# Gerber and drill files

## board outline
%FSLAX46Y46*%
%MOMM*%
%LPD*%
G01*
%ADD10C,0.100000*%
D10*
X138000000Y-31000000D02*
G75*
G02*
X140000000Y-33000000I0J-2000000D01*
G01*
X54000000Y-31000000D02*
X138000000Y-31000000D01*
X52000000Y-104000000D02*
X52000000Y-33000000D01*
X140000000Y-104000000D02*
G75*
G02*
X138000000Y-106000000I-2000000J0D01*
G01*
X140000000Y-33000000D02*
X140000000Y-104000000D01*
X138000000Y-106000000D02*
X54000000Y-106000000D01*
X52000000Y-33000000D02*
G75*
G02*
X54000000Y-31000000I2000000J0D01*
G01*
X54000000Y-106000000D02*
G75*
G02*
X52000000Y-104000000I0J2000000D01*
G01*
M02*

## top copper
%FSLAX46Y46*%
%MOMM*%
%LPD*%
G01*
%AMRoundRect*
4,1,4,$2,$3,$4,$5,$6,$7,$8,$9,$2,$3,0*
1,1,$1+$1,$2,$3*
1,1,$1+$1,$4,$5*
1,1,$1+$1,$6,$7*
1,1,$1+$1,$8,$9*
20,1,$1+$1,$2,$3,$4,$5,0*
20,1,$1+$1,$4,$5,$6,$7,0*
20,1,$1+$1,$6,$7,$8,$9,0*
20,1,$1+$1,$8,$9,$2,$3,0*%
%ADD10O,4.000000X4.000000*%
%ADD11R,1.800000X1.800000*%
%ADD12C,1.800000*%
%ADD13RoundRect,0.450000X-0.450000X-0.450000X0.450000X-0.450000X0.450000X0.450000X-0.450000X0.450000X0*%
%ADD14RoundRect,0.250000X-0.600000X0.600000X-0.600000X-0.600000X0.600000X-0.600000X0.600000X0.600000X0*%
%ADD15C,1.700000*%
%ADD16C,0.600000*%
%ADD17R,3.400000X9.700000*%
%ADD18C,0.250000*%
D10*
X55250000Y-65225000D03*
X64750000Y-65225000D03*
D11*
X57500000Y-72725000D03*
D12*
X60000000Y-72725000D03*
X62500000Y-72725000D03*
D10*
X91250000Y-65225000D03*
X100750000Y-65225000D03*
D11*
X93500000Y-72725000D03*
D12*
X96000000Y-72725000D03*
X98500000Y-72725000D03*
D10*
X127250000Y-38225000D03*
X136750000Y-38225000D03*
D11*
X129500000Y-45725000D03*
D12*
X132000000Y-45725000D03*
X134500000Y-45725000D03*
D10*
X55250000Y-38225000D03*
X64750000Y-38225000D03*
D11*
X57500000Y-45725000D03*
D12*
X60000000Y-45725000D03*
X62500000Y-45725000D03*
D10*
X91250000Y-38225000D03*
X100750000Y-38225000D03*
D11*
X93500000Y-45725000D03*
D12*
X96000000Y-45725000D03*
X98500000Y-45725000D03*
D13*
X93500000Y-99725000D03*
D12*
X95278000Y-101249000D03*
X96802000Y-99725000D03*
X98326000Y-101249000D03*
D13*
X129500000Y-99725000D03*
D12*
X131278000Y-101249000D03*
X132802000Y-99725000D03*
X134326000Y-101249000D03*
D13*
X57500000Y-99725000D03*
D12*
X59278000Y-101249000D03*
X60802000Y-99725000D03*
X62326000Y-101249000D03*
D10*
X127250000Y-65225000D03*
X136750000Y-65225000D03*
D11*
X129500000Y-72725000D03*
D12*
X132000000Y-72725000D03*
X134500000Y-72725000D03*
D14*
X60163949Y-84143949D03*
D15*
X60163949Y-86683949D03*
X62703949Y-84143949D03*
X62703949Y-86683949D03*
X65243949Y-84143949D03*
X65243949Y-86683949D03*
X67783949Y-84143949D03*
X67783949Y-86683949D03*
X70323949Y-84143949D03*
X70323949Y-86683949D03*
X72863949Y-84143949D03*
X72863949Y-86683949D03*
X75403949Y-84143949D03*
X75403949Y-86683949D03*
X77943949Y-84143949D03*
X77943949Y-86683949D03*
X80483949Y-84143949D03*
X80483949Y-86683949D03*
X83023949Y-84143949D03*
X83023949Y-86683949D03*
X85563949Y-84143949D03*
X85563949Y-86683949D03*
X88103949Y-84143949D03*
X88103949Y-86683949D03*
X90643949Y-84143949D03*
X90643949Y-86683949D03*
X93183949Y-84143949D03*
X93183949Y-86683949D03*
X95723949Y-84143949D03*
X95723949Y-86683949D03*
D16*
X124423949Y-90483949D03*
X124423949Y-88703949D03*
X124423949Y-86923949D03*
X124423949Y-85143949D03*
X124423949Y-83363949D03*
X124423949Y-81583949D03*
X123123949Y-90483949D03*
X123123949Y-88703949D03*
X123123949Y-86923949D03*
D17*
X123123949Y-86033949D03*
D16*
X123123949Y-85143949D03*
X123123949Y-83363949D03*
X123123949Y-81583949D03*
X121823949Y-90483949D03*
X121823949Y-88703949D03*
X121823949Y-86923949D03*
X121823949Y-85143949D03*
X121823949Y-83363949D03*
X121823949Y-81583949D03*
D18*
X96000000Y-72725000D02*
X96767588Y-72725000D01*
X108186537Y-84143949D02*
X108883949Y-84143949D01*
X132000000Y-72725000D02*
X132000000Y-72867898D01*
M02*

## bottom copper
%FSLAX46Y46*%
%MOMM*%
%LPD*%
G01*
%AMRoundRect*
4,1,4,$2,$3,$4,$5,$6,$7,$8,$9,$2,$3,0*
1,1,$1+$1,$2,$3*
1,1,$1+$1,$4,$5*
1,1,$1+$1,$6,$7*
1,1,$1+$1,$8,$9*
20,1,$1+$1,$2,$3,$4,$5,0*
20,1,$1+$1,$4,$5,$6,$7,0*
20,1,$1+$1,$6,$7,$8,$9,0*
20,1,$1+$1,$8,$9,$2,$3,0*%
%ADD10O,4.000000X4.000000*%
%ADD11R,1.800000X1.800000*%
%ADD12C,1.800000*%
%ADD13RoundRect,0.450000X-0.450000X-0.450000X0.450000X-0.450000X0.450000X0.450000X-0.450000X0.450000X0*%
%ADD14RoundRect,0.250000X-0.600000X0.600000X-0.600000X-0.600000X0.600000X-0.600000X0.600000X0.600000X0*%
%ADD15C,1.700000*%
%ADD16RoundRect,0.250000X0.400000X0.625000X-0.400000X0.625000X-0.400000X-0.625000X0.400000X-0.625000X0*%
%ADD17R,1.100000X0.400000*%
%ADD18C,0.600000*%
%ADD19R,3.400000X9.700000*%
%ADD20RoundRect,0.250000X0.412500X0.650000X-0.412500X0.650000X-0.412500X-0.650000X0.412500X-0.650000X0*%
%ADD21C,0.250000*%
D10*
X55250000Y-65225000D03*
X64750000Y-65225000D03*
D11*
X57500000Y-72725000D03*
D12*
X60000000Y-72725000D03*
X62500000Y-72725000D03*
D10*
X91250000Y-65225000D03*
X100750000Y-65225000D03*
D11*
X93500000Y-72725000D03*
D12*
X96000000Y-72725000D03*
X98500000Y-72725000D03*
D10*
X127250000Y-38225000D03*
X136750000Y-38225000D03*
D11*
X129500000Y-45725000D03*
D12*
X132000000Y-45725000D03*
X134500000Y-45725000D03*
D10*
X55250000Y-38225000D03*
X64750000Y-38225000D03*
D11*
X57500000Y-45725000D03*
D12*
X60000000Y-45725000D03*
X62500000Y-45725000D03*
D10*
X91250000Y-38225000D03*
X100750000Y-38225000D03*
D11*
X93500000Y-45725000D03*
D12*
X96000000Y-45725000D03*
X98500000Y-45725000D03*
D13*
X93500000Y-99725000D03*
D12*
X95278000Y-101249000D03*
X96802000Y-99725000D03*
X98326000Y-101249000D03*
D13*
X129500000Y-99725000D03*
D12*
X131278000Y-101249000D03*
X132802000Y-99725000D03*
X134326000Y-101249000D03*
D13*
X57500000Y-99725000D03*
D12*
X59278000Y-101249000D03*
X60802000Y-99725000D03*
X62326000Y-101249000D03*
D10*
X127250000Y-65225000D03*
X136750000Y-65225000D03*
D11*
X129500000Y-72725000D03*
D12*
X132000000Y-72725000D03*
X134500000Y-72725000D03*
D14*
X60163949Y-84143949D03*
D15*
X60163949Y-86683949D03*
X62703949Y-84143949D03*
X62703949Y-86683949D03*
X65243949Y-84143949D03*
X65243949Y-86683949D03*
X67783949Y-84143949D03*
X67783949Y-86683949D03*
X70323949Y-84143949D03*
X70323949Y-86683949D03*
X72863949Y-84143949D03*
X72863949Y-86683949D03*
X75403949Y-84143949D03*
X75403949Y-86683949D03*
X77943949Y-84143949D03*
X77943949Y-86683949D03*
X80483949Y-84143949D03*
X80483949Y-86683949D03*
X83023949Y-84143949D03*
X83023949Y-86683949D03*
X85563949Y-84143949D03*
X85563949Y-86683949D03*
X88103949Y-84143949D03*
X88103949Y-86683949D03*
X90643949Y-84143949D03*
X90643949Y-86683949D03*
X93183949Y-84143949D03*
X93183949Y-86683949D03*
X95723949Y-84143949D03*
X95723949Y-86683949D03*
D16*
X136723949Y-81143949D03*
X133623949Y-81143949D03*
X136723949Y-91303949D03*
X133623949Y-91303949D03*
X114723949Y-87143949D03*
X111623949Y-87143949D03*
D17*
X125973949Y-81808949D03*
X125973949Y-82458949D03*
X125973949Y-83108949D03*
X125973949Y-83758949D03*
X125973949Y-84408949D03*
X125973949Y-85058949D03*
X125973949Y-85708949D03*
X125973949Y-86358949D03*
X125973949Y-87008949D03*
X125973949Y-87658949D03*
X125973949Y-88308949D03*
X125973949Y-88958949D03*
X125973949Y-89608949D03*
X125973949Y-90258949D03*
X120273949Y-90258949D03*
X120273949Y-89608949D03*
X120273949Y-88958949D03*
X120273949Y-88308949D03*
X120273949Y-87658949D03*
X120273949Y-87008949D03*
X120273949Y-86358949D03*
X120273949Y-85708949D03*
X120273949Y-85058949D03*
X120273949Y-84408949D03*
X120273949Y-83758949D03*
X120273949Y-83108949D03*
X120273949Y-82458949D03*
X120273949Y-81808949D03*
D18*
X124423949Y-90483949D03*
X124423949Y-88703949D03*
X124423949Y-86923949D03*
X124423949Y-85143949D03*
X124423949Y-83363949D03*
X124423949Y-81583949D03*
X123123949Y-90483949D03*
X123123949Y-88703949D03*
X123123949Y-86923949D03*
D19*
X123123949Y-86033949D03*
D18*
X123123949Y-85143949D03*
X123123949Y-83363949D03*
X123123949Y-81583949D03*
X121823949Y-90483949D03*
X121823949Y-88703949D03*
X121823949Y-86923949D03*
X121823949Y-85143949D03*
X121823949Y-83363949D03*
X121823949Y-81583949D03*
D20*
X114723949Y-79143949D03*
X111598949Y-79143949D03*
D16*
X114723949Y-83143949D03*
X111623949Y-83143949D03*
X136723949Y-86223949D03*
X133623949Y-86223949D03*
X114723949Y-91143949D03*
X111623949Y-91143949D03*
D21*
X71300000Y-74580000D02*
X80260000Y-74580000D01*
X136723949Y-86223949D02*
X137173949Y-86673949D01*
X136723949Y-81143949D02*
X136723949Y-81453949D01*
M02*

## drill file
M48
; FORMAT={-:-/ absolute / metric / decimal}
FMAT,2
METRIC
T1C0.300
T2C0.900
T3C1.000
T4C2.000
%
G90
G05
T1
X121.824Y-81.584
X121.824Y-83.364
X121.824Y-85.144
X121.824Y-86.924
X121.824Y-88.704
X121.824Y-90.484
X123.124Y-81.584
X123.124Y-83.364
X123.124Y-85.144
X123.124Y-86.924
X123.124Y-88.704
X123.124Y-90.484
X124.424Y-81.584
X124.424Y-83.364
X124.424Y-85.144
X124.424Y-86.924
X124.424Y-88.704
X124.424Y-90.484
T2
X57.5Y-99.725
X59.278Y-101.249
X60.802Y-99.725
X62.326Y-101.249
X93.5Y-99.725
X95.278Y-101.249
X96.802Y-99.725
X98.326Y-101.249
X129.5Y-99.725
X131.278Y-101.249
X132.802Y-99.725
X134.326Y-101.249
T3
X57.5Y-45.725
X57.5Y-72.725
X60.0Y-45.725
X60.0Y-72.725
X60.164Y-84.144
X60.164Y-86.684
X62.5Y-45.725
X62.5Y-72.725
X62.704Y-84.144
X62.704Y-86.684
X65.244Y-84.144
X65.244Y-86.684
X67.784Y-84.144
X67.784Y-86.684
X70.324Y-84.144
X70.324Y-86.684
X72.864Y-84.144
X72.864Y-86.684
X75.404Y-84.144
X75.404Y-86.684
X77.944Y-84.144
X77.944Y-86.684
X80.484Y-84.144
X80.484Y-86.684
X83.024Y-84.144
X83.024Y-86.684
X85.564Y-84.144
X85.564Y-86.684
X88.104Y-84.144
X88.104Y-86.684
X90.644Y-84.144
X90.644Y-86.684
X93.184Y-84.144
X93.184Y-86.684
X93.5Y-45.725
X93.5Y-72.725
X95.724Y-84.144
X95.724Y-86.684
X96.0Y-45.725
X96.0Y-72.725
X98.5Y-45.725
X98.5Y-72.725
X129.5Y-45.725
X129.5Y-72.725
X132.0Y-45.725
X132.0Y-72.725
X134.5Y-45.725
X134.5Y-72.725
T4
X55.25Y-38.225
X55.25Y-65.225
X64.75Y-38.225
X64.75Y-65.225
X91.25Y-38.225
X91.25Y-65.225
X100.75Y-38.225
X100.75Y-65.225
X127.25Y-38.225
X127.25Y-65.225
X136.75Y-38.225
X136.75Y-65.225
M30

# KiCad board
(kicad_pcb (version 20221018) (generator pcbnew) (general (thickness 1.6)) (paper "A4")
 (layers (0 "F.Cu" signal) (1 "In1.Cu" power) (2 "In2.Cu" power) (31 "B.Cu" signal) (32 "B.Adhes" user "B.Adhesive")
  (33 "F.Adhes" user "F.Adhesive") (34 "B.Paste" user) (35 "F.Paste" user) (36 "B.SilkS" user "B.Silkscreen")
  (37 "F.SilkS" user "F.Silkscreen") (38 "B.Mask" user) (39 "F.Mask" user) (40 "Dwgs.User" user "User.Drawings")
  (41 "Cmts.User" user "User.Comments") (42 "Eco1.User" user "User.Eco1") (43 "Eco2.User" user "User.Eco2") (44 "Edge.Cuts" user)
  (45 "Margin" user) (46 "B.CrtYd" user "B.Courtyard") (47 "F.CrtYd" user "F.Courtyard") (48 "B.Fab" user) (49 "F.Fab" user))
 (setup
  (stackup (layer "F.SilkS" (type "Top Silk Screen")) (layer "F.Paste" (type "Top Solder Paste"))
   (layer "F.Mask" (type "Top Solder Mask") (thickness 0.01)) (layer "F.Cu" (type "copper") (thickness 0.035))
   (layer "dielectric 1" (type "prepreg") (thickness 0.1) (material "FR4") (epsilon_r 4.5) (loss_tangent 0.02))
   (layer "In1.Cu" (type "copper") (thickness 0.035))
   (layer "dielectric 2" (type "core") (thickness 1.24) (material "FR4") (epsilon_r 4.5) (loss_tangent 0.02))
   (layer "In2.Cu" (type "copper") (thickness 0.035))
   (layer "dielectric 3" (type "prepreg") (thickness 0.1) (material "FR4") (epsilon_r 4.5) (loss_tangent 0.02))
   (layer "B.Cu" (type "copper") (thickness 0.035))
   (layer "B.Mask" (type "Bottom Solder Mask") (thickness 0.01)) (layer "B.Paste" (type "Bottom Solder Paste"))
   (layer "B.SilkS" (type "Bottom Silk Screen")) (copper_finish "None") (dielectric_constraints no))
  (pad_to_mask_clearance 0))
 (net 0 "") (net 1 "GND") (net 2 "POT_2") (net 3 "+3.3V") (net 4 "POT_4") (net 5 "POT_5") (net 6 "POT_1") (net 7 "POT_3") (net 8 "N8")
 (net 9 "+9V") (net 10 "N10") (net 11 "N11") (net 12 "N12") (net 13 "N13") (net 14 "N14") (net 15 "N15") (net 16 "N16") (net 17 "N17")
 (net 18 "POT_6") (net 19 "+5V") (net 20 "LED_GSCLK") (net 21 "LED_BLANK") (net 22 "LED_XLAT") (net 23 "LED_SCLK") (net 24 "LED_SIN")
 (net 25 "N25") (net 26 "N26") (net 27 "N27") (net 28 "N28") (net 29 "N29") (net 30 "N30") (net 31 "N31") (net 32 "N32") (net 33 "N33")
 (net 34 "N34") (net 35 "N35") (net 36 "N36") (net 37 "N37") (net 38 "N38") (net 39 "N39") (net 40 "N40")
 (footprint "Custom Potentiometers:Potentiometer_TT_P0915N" (layer "F.Cu") (at 57.5 72.725)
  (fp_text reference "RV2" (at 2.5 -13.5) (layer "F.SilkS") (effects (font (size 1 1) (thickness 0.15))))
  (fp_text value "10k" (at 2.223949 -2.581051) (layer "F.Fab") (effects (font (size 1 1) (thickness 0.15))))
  (pad "" thru_hole oval (at -2.25 -7.5) (size 4 4) (drill 2) (layers "*.Cu" "*.Mask"))
  (pad "" thru_hole oval (at 7.25 -7.5) (size 4 4) (drill 2) (layers "*.Cu" "*.Mask"))
  (pad "1" thru_hole rect (at 0 0) (size 1.8 1.8) (drill 1) (layers "*.Cu" "*.Mask") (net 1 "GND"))
  (pad "2" thru_hole circle (at 2.5 0) (size 1.8 1.8) (drill 1) (layers "*.Cu" "*.Mask") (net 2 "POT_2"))
  (pad "3" thru_hole circle (at 5 0) (size 1.8 1.8) (drill 1) (layers "*.Cu" "*.Mask") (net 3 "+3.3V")))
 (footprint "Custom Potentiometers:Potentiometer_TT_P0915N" (layer "F.Cu") (at 93.5 72.725)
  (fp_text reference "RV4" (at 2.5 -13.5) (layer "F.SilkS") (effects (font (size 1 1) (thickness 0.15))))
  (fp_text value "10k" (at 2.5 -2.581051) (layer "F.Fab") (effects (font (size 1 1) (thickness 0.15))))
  (pad "" thru_hole oval (at -2.25 -7.5) (size 4 4) (drill 2) (layers "*.Cu" "*.Mask"))
  (pad "" thru_hole oval (at 7.25 -7.5) (size 4 4) (drill 2) (layers "*.Cu" "*.Mask"))
  (pad "1" thru_hole rect (at 0 0) (size 1.8 1.8) (drill 1) (layers "*.Cu" "*.Mask") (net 1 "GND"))
  (pad "2" thru_hole circle (at 2.5 0) (size 1.8 1.8) (drill 1) (layers "*.Cu" "*.Mask") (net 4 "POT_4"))
  (pad "3" thru_hole circle (at 5 0) (size 1.8 1.8) (drill 1) (layers "*.Cu" "*.Mask") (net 3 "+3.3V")))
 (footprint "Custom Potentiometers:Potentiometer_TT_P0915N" (layer "F.Cu") (at 129.5 45.725)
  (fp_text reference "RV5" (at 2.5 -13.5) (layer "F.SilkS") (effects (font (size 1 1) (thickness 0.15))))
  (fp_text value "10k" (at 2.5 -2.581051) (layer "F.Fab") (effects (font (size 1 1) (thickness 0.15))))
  (pad "" thru_hole oval (at -2.25 -7.5) (size 4 4) (drill 2) (layers "*.Cu" "*.Mask"))
  (pad "" thru_hole oval (at 7.25 -7.5) (size 4 4) (drill 2) (layers "*.Cu" "*.Mask"))
  (pad "1" thru_hole rect (at 0 0) (size 1.8 1.8) (drill 1) (layers "*.Cu" "*.Mask") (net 1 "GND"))
  (pad "2" thru_hole circle (at 2.5 0) (size 1.8 1.8) (drill 1) (layers "*.Cu" "*.Mask") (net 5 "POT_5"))
  (pad "3" thru_hole circle (at 5 0) (size 1.8 1.8) (drill 1) (layers "*.Cu" "*.Mask") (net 3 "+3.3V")))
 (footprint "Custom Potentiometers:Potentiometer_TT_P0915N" (layer "F.Cu") (at 57.5 45.725)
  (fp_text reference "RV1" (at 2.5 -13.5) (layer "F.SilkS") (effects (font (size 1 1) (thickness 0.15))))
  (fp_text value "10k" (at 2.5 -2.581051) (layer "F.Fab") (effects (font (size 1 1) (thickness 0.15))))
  (pad "" thru_hole oval (at -2.25 -7.5) (size 4 4) (drill 2) (layers "*.Cu" "*.Mask"))
  (pad "" thru_hole oval (at 7.25 -7.5) (size 4 4) (drill 2) (layers "*.Cu" "*.Mask"))
  (pad "1" thru_hole rect (at 0 0) (size 1.8 1.8) (drill 1) (layers "*.Cu" "*.Mask") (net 1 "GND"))
  (pad "2" thru_hole circle (at 2.5 0) (size 1.8 1.8) (drill 1) (layers "*.Cu" "*.Mask") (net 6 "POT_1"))
  (pad "3" thru_hole circle (at 5 0) (size 1.8 1.8) (drill 1) (layers "*.Cu" "*.Mask") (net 3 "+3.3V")))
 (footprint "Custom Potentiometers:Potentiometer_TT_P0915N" (layer "F.Cu") (at 93.5 45.725)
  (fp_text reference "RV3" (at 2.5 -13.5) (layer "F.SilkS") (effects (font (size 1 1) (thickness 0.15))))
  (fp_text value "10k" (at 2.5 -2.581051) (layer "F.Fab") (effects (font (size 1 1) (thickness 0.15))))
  (pad "" thru_hole oval (at -2.25 -7.5) (size 4 4) (drill 2) (layers "*.Cu" "*.Mask"))
  (pad "" thru_hole oval (at 7.25 -7.5) (size 4 4) (drill 2) (layers "*.Cu" "*.Mask"))
  (pad "1" thru_hole rect (at 0 0) (size 1.8 1.8) (drill 1) (layers "*.Cu" "*.Mask") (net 1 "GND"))
  (pad "2" thru_hole circle (at 2.5 0) (size 1.8 1.8) (drill 1) (layers "*.Cu" "*.Mask") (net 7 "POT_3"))
  (pad "3" thru_hole circle (at 5 0) (size 1.8 1.8) (drill 1) (layers "*.Cu" "*.Mask") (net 3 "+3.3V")))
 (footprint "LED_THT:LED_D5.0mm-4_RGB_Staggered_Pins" (layer "F.Cu") (at 93.5 99.725)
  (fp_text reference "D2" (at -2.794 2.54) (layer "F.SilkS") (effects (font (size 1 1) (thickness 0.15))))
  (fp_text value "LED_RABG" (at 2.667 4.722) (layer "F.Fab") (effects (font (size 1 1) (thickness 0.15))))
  (pad "1" thru_hole roundrect (at 0 0) (size 1.8 1.8) (drill 0.9) (layers "*.Cu" "*.Mask") (roundrect_rratio 0.25) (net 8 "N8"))
  (pad "2" thru_hole circle (at 1.778 1.524) (size 1.8 1.8) (drill 0.9) (layers "*.Cu" "*.Mask") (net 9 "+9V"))
  (pad "3" thru_hole circle (at 3.302 0) (size 1.8 1.8) (drill 0.9) (layers "*.Cu" "*.Mask") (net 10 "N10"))
  (pad "4" thru_hole circle (at 4.826 1.524) (size 1.8 1.8) (drill 0.9) (layers "*.Cu" "*.Mask") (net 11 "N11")))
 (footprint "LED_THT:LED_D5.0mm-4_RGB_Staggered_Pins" (layer "F.Cu") (at 129.5 99.725)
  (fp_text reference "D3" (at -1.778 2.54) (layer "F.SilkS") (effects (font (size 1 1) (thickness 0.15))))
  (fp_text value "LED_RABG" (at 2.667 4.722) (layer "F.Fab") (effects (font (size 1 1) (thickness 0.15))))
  (pad "1" thru_hole roundrect (at 0 0) (size 1.8 1.8) (drill 0.9) (layers "*.Cu" "*.Mask") (roundrect_rratio 0.25) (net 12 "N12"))
  (pad "2" thru_hole circle (at 1.778 1.524) (size 1.8 1.8) (drill 0.9) (layers "*.Cu" "*.Mask") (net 9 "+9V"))
  (pad "3" thru_hole circle (at 3.302 0) (size 1.8 1.8) (drill 0.9) (layers "*.Cu" "*.Mask") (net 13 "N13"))
  (pad "4" thru_hole circle (at 4.826 1.524) (size 1.8 1.8) (drill 0.9) (layers "*.Cu" "*.Mask") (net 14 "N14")))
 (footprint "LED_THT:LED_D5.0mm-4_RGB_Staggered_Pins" (layer "F.Cu") (at 57.5 99.725)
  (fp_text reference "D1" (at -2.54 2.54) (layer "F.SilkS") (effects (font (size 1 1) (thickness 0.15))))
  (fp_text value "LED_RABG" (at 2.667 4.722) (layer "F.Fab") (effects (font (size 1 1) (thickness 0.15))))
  (pad "1" thru_hole roundrect (at 0 0) (size 1.8 1.8) (drill 0.9) (layers "*.Cu" "*.Mask") (roundrect_rratio 0.25) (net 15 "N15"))
  (pad "2" thru_hole circle (at 1.778 1.524) (size 1.8 1.8) (drill 0.9) (layers "*.Cu" "*.Mask") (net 9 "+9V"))
  (pad "3" thru_hole circle (at 3.302 0) (size 1.8 1.8) (drill 0.9) (layers "*.Cu" "*.Mask") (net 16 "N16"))
  (pad "4" thru_hole circle (at 4.826 1.524) (size 1.8 1.8) (drill 0.9) (layers "*.Cu" "*.Mask") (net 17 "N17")))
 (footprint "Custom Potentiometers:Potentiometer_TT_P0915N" (layer "F.Cu") (at 129.5 72.725)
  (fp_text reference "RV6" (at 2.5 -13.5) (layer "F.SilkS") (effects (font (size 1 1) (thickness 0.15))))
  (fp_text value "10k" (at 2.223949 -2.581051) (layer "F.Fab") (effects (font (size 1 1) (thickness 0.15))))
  (pad "" thru_hole oval (at -2.25 -7.5) (size 4 4) (drill 2) (layers "*.Cu" "*.Mask"))
  (pad "" thru_hole oval (at 7.25 -7.5) (size 4 4) (drill 2) (layers "*.Cu" "*.Mask"))
  (pad "1" thru_hole rect (at 0 0) (size 1.8 1.8) (drill 1) (layers "*.Cu" "*.Mask") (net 1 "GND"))
  (pad "2" thru_hole circle (at 2.5 0) (size 1.8 1.8) (drill 1) (layers "*.Cu" "*.Mask") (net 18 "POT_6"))
  (pad "3" thru_hole circle (at 5 0) (size 1.8 1.8) (drill 1) (layers "*.Cu" "*.Mask") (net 3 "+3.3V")))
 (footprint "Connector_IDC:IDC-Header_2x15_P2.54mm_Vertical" (layer "B.Cu") (at 60.163949 84.143949 -90)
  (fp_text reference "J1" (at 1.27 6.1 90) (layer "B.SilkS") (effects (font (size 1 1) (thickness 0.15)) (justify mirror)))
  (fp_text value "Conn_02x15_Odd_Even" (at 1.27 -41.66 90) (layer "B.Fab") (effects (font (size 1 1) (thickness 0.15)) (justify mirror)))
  (pad "1" thru_hole roundrect (at 0 0 270) (size 1.7 1.7) (drill 1) (layers "*.Cu" "*.Mask") (roundrect_rratio 0.147059) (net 9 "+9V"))
  (pad "2" thru_hole circle (at 2.54 0 270) (size 1.7 1.7) (drill 1) (layers "*.Cu" "*.Mask") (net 1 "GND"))
  (pad "3" thru_hole circle (at 0 -2.54 270) (size 1.7 1.7) (drill 1) (layers "*.Cu" "*.Mask") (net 9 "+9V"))
  (pad "4" thru_hole circle (at 2.54 -2.54 270) (size 1.7 1.7) (drill 1) (layers "*.Cu" "*.Mask") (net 1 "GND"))
  (pad "5" thru_hole circle (at 0 -5.08 270) (size 1.7 1.7) (drill 1) (layers "*.Cu" "*.Mask") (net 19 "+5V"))
  (pad "6" thru_hole circle (at 2.54 -5.08 270) (size 1.7 1.7) (drill 1) (layers "*.Cu" "*.Mask") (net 1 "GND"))
  (pad "7" thru_hole circle (at 0 -7.62 270) (size 1.7 1.7) (drill 1) (layers "*.Cu" "*.Mask") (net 3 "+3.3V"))
  (pad "8" thru_hole circle (at 2.54 -7.62 270) (size 1.7 1.7) (drill 1) (layers "*.Cu" "*.Mask") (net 1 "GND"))
  (pad "9" thru_hole circle (at 0 -10.16 270) (size 1.7 1.7) (drill 1) (layers "*.Cu" "*.Mask") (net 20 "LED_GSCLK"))
  (pad "10" thru_hole circle (at 2.54 -10.16 270) (size 1.7 1.7) (drill 1) (layers "*.Cu" "*.Mask") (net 1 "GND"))
  (pad "11" thru_hole circle (at 0 -12.7 270) (size 1.7 1.7) (drill 1) (layers "*.Cu" "*.Mask") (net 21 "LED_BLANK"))
  (pad "12" thru_hole circle (at 2.54 -12.7 270) (size 1.7 1.7) (drill 1) (layers "*.Cu" "*.Mask") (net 1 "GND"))
  (pad "13" thru_hole circle (at 0 -15.24 270) (size 1.7 1.7) (drill 1) (layers "*.Cu" "*.Mask") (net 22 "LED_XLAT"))
  (pad "14" thru_hole circle (at 2.54 -15.24 270) (size 1.7 1.7) (drill 1) (layers "*.Cu" "*.Mask") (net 1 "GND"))
  (pad "15" thru_hole circle (at 0 -17.78 270) (size 1.7 1.7) (drill 1) (layers "*.Cu" "*.Mask") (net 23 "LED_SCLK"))
  (pad "16" thru_hole circle (at 2.54 -17.78 270) (size 1.7 1.7) (drill 1) (layers "*.Cu" "*.Mask") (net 1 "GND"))
  (pad "17" thru_hole circle (at 0 -20.32 270) (size 1.7 1.7) (drill 1) (layers "*.Cu" "*.Mask") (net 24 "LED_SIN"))
  (pad "18" thru_hole circle (at 2.54 -20.32 270) (size 1.7 1.7) (drill 1) (layers "*.Cu" "*.Mask") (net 1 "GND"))
  (pad "19" thru_hole circle (at 0 -22.86 270) (size 1.7 1.7) (drill 1) (layers "*.Cu" "*.Mask") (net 6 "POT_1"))
  (pad "20" thru_hole circle (at 2.54 -22.86 270) (size 1.7 1.7) (drill 1) (layers "*.Cu" "*.Mask") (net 1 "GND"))
  (pad "21" thru_hole circle (at 0 -25.4 270) (size 1.7 1.7) (drill 1) (layers "*.Cu" "*.Mask") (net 2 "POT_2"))
  (pad "22" thru_hole circle (at 2.54 -25.4 270) (size 1.7 1.7) (drill 1) (layers "*.Cu" "*.Mask") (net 1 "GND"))
  (pad "23" thru_hole circle (at 0 -27.94 270) (size 1.7 1.7) (drill 1) (layers "*.Cu" "*.Mask") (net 7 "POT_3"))
  (pad "24" thru_hole circle (at 2.54 -27.94 270) (size 1.7 1.7) (drill 1) (layers "*.Cu" "*.Mask") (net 1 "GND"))
  (pad "25" thru_hole circle (at 0 -30.48 270) (size 1.7 1.7) (drill 1) (layers "*.Cu" "*.Mask") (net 4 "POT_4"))
  (pad "26" thru_hole circle (at 2.54 -30.48 270) (size 1.7 1.7) (drill 1) (layers "*.Cu" "*.Mask") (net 1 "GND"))
  (pad "27" thru_hole circle (at 0 -33.02 270) (size 1.7 1.7) (drill 1) (layers "*.Cu" "*.Mask") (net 5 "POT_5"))
  (pad "28" thru_hole circle (at 2.54 -33.02 270) (size 1.7 1.7) (drill 1) (layers "*.Cu" "*.Mask") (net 1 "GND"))
  (pad "29" thru_hole circle (at 0 -35.56 270) (size 1.7 1.7) (drill 1) (layers "*.Cu" "*.Mask") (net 18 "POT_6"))
  (pad "30" thru_hole circle (at 2.54 -35.56 270) (size 1.7 1.7) (drill 1) (layers "*.Cu" "*.Mask") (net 1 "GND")))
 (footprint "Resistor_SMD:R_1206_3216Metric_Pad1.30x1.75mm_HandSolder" (layer "B.Cu") (at 135.173949 81.143949 180)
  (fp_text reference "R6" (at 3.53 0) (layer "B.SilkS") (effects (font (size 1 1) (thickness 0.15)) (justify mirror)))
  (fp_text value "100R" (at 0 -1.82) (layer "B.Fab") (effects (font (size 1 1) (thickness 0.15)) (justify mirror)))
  (pad "1" smd roundrect (at -1.55 0 180) (size 1.3 1.75) (layers "B.Cu" "B.Paste" "B.Mask") (roundrect_rratio 0.192308) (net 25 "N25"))
  (pad "2" smd roundrect (at 1.55 0 180) (size 1.3 1.75) (layers "B.Cu" "B.Paste" "B.Mask") (roundrect_rratio 0.192308) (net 24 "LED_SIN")))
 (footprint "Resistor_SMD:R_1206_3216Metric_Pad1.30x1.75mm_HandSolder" (layer "B.Cu") (at 135.173949 91.303949 180)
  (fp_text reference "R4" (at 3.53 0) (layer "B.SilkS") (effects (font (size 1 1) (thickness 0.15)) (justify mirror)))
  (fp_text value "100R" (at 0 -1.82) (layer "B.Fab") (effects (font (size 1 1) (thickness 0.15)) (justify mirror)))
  (pad "1" smd roundrect (at -1.55 0 180) (size 1.3 1.75) (layers "B.Cu" "B.Paste" "B.Mask") (roundrect_rratio 0.192308) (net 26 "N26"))
  (pad "2" smd roundrect (at 1.55 0 180) (size 1.3 1.75) (layers "B.Cu" "B.Paste" "B.Mask") (roundrect_rratio 0.192308) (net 22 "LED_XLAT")))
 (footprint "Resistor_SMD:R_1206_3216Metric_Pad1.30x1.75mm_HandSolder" (layer "B.Cu") (at 113.173949 87.143949 180)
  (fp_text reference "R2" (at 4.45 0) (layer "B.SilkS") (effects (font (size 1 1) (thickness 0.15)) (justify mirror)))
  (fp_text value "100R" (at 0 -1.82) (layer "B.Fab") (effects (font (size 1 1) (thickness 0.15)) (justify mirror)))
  (pad "1" smd roundrect (at -1.55 0 180) (size 1.3 1.75) (layers "B.Cu" "B.Paste" "B.Mask") (roundrect_rratio 0.192308) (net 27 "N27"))
  (pad "2" smd roundrect (at 1.55 0 180) (size 1.3 1.75) (layers "B.Cu" "B.Paste" "B.Mask") (roundrect_rratio 0.192308) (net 20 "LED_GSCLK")))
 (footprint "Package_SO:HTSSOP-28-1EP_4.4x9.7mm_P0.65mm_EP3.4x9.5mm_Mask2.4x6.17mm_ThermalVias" (layer "B.Cu") (at 123.123949 86.033949 180)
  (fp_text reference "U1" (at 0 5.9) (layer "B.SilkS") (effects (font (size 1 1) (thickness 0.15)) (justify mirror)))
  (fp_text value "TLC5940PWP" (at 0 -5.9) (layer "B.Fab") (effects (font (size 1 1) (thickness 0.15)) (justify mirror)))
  (pad "" smd rect (at -0.6 -1.78 180) (size 0.9 1.4) (layers "B.Paste"))
  (pad "" smd rect (at -0.6 0 180) (size 0.9 1.4) (layers "B.Paste"))
  (pad "" smd rect (at -0.6 1.78 180) (size 0.9 1.4) (layers "B.Paste"))
  (pad "" smd rect (at 0 0 180) (size 2.4 6.17) (layers "B.Mask"))
  (pad "" smd rect (at 0.6 -1.78 180) (size 0.9 1.4) (layers "B.Paste"))
  (pad "" smd rect (at 0.6 0 180) (size 0.9 1.4) (layers "B.Paste"))
  (pad "" smd rect (at 0.6 1.78 180) (size 0.9 1.4) (layers "B.Paste"))
  (pad "1" smd rect (at -2.85 4.225 180) (size 1.1 0.4) (layers "B.Cu" "B.Paste" "B.Mask") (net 1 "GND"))
  (pad "2" smd rect (at -2.85 3.575 180) (size 1.1 0.4) (layers "B.Cu" "B.Paste" "B.Mask") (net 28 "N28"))
  (pad "3" smd rect (at -2.85 2.925 180) (size 1.1 0.4) (layers "B.Cu" "B.Paste" "B.Mask") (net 26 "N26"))
  (pad "4" smd rect (at -2.85 2.275 180) (size 1.1 0.4) (layers "B.Cu" "B.Paste" "B.Mask") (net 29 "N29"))
  (pad "5" smd rect (at -2.85 1.625 180) (size 1.1 0.4) (layers "B.Cu" "B.Paste" "B.Mask") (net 25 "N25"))
  (pad "6" smd rect (at -2.85 0.975 180) (size 1.1 0.4) (layers "B.Cu" "B.Paste" "B.Mask") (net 1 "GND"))
  (pad "7" smd rect (at -2.85 0.325 180) (size 1.1 0.4) (layers "B.Cu" "B.Paste" "B.Mask") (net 15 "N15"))
  (pad "8" smd rect (at -2.85 -0.325 180) (size 1.1 0.4) (layers "B.Cu" "B.Paste" "B.Mask") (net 17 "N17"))
  (pad "9" smd rect (at -2.85 -0.975 180) (size 1.1 0.4) (layers "B.Cu" "B.Paste" "B.Mask") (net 16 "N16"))
  (pad "10" smd rect (at -2.85 -1.625 180) (size 1.1 0.4) (layers "B.Cu" "B.Paste" "B.Mask") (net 8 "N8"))
  (pad "11" smd rect (at -2.85 -2.275 180) (size 1.1 0.4) (layers "B.Cu" "B.Paste" "B.Mask") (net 11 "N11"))
  (pad "12" smd rect (at -2.85 -2.925 180) (size 1.1 0.4) (layers "B.Cu" "B.Paste" "B.Mask") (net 10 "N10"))
  (pad "13" smd rect (at -2.85 -3.575 180) (size 1.1 0.4) (layers "B.Cu" "B.Paste" "B.Mask") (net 12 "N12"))
  (pad "14" smd rect (at -2.85 -4.225 180) (size 1.1 0.4) (layers "B.Cu" "B.Paste" "B.Mask") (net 14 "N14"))
  (pad "15" smd rect (at 2.85 -4.225 180) (size 1.1 0.4) (layers "B.Cu" "B.Paste" "B.Mask") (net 13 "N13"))
  (pad "16" smd rect (at 2.85 -3.575 180) (size 1.1 0.4) (layers "B.Cu" "B.Paste" "B.Mask") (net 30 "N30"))
  (pad "17" smd rect (at 2.85 -2.925 180) (size 1.1 0.4) (layers "B.Cu" "B.Paste" "B.Mask") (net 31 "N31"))
  (pad "18" smd rect (at 2.85 -2.275 180) (size 1.1 0.4) (layers "B.Cu" "B.Paste" "B.Mask") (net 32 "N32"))
  (pad "19" smd rect (at 2.85 -1.625 180) (size 1.1 0.4) (layers "B.Cu" "B.Paste" "B.Mask") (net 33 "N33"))
  (pad "20" smd rect (at 2.85 -0.975 180) (size 1.1 0.4) (layers "B.Cu" "B.Paste" "B.Mask") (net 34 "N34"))
  (pad "21" smd rect (at 2.85 -0.325 180) (size 1.1 0.4) (layers "B.Cu" "B.Paste" "B.Mask") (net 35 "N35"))
  (pad "22" smd rect (at 2.85 0.325 180) (size 1.1 0.4) (layers "B.Cu" "B.Paste" "B.Mask") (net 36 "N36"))
  (pad "23" smd rect (at 2.85 0.975 180) (size 1.1 0.4) (layers "B.Cu" "B.Paste" "B.Mask") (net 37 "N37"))
  (pad "24" smd rect (at 2.85 1.625 180) (size 1.1 0.4) (layers "B.Cu" "B.Paste" "B.Mask") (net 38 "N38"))
  (pad "25" smd rect (at 2.85 2.275 180) (size 1.1 0.4) (layers "B.Cu" "B.Paste" "B.Mask") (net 27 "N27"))
  (pad "26" smd rect (at 2.85 2.925 180) (size 1.1 0.4) (layers "B.Cu" "B.Paste" "B.Mask") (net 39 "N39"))
  (pad "27" smd rect (at 2.85 3.575 180) (size 1.1 0.4) (layers "B.Cu" "B.Paste" "B.Mask") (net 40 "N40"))
  (pad "28" smd rect (at 2.85 4.225 180) (size 1.1 0.4) (layers "B.Cu" "B.Paste" "B.Mask") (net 3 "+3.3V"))
  (pad "29" thru_hole circle (at -1.3 -4.45 180) (size 0.6 0.6) (drill 0.3) (layers "*.Cu") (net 1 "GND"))
  (pad "29" thru_hole circle (at -1.3 -2.67 180) (size 0.6 0.6) (drill 0.3) (layers "*.Cu") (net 1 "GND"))
  (pad "29" thru_hole circle (at -1.3 -0.89 180) (size 0.6 0.6) (drill 0.3) (layers "*.Cu") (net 1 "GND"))
  (pad "29" thru_hole circle (at -1.3 0.89 180) (size 0.6 0.6) (drill 0.3) (layers "*.Cu") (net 1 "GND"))
  (pad "29" thru_hole circle (at -1.3 2.67 180) (size 0.6 0.6) (drill 0.3) (layers "*.Cu") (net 1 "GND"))
  (pad "29" thru_hole circle (at -1.3 4.45 180) (size 0.6 0.6) (drill 0.3) (layers "*.Cu") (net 1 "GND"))
  (pad "29" thru_hole circle (at 0 -4.45 180) (size 0.6 0.6) (drill 0.3) (layers "*.Cu") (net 1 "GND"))
  (pad "29" thru_hole circle (at 0 -2.67 180) (size 0.6 0.6) (drill 0.3) (layers "*.Cu") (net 1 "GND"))
  (pad "29" thru_hole circle (at 0 -0.89 180) (size 0.6 0.6) (drill 0.3) (layers "*.Cu") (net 1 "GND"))
  (pad "29" smd rect (at 0 0 180) (size 3.4 9.7) (layers "F.Cu") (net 1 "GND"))
  (pad "29" smd rect (at 0 0 180) (size 3.4 9.7) (layers "B.Cu") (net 1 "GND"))
  (pad "29" thru_hole circle (at 0 0.89 180) (size 0.6 0.6) (drill 0.3) (layers "*.Cu") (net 1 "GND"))
  (pad "29" thru_hole circle (at 0 2.67 180) (size 0.6 0.6) (drill 0.3) (layers "*.Cu") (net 1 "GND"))
  (pad "29" thru_hole circle (at 0 4.45 180) (size 0.6 0.6) (drill 0.3) (layers "*.Cu") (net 1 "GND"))
  (pad "29" thru_hole circle (at 1.3 -4.45 180) (size 0.6 0.6) (drill 0.3) (layers "*.Cu") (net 1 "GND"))
  (pad "29" thru_hole circle (at 1.3 -2.67 180) (size 0.6 0.6) (drill 0.3) (layers "*.Cu") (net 1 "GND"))
  (pad "29" thru_hole circle (at 1.3 -0.89 180) (size 0.6 0.6) (drill 0.3) (layers "*.Cu") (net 1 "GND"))
  (pad "29" thru_hole circle (at 1.3 0.89 180) (size 0.6 0.6) (drill 0.3) (layers "*.Cu") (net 1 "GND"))
  (pad "29" thru_hole circle (at 1.3 2.67 180) (size 0.6 0.6) (drill 0.3) (layers "*.Cu") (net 1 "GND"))
  (pad "29" thru_hole circle (at 1.3 4.45 180) (size 0.6 0.6) (drill 0.3) (layers "*.Cu") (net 1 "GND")))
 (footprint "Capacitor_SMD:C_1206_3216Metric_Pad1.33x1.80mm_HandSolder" (layer "B.Cu") (at 113.161449 79.143949 180)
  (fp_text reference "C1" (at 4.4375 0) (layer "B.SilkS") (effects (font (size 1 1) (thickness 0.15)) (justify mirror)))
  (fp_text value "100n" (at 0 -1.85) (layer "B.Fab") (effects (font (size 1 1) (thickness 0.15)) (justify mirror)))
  (pad "1" smd roundrect (at -1.5625 0 180) (size 1.325 1.8) (layers "B.Cu" "B.Paste" "B.Mask") (roundrect_rratio 0.188679) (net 1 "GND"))
  (pad "2" smd roundrect (at 1.5625 0 180) (size 1.325 1.8) (layers "B.Cu" "B.Paste" "B.Mask") (roundrect_rratio 0.188679) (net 3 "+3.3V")))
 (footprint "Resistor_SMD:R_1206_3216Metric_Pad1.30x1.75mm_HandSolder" (layer "B.Cu") (at 113.173949 83.143949 180)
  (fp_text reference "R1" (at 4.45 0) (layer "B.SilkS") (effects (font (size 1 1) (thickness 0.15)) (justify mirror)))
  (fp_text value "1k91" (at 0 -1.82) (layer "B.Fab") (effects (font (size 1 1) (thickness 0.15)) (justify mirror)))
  (pad "1" smd roundrect (at -1.55 0 180) (size 1.3 1.75) (layers "B.Cu" "B.Paste" "B.Mask") (roundrect_rratio 0.192308) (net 40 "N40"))
  (pad "2" smd roundrect (at 1.55 0 180) (size 1.3 1.75) (layers "B.Cu" "B.Paste" "B.Mask") (roundrect_rratio 0.192308) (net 1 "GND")))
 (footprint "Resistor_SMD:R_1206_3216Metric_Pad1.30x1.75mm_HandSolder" (layer "B.Cu") (at 135.173949 86.223949 180)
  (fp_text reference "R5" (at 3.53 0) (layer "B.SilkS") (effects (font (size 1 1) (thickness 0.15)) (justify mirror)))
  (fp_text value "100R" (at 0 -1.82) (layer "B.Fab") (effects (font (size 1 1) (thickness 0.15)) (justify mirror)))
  (pad "1" smd roundrect (at -1.55 0 180) (size 1.3 1.75) (layers "B.Cu" "B.Paste" "B.Mask") (roundrect_rratio 0.192308) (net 29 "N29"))
  (pad "2" smd roundrect (at 1.55 0 180) (size 1.3 1.75) (layers "B.Cu" "B.Paste" "B.Mask") (roundrect_rratio 0.192308) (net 23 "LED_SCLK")))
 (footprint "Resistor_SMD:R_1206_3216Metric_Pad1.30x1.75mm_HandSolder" (layer "B.Cu") (at 113.173949 91.143949 180)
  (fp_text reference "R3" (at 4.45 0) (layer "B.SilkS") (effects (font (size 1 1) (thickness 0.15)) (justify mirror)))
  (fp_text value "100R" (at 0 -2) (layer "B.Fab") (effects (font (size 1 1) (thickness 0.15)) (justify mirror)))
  (pad "1" smd roundrect (at -1.55 0 180) (size 1.3 1.75) (layers "B.Cu" "B.Paste" "B.Mask") (roundrect_rratio 0.192308) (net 28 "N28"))
  (pad "2" smd roundrect (at 1.55 0 180) (size 1.3 1.75) (layers "B.Cu" "B.Paste" "B.Mask") (roundrect_rratio 0.192308) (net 21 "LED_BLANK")))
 (gr_arc (start 138 31) (mid 139.414214 31.585786) (end 140 33) (stroke (width 0.1) (type default)) (layer "Edge.Cuts"))
 (gr_line (start 54 31) (end 138 31) (stroke (width 0.1) (type default)) (layer "Edge.Cuts"))
 (gr_line (start 52 104) (end 52 33) (stroke (width 0.1) (type default)) (layer "Edge.Cuts"))
 (gr_arc (start 140 104) (mid 139.414214 105.414214) (end 138 106) (stroke (width 0.1) (type default)) (layer "Edge.Cuts"))
 (gr_line (start 140 33) (end 140 104) (stroke (width 0.1) (type default)) (layer "Edge.Cuts"))
 (gr_line (start 138 106) (end 54 106) (stroke (width 0.1) (type default)) (layer "Edge.Cuts"))
 (gr_arc (start 52 33) (mid 52.585786 31.585786) (end 54 31) (stroke (width 0.1) (type default)) (layer "Edge.Cuts"))
 (gr_arc (start 54 106) (mid 52.585786 105.414214) (end 52 104) (stroke (width 0.1) (type default)) (layer "Edge.Cuts"))
 (segment (start 71.3 74.58) (end 80.26 74.58) (width 0.25) (layer "B.Cu") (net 27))
 (segment (start 136.723949 86.223949) (end 137.173949 86.673949) (width 0.25) (layer "B.Cu") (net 29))
 (segment (start 136.723949 81.143949) (end 136.723949 81.453949) (width 0.25) (layer "B.Cu") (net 25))
 (segment (start 96 72.725) (end 96.767588 72.725) (width 0.25) (layer "F.Cu") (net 4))
 (segment (start 108.186537 84.143949) (end 108.883949 84.143949) (width 0.25) (layer "F.Cu") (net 4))
 (segment (start 132 72.725) (end 132 72.867898) (width 0.25) (layer "F.Cu") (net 18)))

